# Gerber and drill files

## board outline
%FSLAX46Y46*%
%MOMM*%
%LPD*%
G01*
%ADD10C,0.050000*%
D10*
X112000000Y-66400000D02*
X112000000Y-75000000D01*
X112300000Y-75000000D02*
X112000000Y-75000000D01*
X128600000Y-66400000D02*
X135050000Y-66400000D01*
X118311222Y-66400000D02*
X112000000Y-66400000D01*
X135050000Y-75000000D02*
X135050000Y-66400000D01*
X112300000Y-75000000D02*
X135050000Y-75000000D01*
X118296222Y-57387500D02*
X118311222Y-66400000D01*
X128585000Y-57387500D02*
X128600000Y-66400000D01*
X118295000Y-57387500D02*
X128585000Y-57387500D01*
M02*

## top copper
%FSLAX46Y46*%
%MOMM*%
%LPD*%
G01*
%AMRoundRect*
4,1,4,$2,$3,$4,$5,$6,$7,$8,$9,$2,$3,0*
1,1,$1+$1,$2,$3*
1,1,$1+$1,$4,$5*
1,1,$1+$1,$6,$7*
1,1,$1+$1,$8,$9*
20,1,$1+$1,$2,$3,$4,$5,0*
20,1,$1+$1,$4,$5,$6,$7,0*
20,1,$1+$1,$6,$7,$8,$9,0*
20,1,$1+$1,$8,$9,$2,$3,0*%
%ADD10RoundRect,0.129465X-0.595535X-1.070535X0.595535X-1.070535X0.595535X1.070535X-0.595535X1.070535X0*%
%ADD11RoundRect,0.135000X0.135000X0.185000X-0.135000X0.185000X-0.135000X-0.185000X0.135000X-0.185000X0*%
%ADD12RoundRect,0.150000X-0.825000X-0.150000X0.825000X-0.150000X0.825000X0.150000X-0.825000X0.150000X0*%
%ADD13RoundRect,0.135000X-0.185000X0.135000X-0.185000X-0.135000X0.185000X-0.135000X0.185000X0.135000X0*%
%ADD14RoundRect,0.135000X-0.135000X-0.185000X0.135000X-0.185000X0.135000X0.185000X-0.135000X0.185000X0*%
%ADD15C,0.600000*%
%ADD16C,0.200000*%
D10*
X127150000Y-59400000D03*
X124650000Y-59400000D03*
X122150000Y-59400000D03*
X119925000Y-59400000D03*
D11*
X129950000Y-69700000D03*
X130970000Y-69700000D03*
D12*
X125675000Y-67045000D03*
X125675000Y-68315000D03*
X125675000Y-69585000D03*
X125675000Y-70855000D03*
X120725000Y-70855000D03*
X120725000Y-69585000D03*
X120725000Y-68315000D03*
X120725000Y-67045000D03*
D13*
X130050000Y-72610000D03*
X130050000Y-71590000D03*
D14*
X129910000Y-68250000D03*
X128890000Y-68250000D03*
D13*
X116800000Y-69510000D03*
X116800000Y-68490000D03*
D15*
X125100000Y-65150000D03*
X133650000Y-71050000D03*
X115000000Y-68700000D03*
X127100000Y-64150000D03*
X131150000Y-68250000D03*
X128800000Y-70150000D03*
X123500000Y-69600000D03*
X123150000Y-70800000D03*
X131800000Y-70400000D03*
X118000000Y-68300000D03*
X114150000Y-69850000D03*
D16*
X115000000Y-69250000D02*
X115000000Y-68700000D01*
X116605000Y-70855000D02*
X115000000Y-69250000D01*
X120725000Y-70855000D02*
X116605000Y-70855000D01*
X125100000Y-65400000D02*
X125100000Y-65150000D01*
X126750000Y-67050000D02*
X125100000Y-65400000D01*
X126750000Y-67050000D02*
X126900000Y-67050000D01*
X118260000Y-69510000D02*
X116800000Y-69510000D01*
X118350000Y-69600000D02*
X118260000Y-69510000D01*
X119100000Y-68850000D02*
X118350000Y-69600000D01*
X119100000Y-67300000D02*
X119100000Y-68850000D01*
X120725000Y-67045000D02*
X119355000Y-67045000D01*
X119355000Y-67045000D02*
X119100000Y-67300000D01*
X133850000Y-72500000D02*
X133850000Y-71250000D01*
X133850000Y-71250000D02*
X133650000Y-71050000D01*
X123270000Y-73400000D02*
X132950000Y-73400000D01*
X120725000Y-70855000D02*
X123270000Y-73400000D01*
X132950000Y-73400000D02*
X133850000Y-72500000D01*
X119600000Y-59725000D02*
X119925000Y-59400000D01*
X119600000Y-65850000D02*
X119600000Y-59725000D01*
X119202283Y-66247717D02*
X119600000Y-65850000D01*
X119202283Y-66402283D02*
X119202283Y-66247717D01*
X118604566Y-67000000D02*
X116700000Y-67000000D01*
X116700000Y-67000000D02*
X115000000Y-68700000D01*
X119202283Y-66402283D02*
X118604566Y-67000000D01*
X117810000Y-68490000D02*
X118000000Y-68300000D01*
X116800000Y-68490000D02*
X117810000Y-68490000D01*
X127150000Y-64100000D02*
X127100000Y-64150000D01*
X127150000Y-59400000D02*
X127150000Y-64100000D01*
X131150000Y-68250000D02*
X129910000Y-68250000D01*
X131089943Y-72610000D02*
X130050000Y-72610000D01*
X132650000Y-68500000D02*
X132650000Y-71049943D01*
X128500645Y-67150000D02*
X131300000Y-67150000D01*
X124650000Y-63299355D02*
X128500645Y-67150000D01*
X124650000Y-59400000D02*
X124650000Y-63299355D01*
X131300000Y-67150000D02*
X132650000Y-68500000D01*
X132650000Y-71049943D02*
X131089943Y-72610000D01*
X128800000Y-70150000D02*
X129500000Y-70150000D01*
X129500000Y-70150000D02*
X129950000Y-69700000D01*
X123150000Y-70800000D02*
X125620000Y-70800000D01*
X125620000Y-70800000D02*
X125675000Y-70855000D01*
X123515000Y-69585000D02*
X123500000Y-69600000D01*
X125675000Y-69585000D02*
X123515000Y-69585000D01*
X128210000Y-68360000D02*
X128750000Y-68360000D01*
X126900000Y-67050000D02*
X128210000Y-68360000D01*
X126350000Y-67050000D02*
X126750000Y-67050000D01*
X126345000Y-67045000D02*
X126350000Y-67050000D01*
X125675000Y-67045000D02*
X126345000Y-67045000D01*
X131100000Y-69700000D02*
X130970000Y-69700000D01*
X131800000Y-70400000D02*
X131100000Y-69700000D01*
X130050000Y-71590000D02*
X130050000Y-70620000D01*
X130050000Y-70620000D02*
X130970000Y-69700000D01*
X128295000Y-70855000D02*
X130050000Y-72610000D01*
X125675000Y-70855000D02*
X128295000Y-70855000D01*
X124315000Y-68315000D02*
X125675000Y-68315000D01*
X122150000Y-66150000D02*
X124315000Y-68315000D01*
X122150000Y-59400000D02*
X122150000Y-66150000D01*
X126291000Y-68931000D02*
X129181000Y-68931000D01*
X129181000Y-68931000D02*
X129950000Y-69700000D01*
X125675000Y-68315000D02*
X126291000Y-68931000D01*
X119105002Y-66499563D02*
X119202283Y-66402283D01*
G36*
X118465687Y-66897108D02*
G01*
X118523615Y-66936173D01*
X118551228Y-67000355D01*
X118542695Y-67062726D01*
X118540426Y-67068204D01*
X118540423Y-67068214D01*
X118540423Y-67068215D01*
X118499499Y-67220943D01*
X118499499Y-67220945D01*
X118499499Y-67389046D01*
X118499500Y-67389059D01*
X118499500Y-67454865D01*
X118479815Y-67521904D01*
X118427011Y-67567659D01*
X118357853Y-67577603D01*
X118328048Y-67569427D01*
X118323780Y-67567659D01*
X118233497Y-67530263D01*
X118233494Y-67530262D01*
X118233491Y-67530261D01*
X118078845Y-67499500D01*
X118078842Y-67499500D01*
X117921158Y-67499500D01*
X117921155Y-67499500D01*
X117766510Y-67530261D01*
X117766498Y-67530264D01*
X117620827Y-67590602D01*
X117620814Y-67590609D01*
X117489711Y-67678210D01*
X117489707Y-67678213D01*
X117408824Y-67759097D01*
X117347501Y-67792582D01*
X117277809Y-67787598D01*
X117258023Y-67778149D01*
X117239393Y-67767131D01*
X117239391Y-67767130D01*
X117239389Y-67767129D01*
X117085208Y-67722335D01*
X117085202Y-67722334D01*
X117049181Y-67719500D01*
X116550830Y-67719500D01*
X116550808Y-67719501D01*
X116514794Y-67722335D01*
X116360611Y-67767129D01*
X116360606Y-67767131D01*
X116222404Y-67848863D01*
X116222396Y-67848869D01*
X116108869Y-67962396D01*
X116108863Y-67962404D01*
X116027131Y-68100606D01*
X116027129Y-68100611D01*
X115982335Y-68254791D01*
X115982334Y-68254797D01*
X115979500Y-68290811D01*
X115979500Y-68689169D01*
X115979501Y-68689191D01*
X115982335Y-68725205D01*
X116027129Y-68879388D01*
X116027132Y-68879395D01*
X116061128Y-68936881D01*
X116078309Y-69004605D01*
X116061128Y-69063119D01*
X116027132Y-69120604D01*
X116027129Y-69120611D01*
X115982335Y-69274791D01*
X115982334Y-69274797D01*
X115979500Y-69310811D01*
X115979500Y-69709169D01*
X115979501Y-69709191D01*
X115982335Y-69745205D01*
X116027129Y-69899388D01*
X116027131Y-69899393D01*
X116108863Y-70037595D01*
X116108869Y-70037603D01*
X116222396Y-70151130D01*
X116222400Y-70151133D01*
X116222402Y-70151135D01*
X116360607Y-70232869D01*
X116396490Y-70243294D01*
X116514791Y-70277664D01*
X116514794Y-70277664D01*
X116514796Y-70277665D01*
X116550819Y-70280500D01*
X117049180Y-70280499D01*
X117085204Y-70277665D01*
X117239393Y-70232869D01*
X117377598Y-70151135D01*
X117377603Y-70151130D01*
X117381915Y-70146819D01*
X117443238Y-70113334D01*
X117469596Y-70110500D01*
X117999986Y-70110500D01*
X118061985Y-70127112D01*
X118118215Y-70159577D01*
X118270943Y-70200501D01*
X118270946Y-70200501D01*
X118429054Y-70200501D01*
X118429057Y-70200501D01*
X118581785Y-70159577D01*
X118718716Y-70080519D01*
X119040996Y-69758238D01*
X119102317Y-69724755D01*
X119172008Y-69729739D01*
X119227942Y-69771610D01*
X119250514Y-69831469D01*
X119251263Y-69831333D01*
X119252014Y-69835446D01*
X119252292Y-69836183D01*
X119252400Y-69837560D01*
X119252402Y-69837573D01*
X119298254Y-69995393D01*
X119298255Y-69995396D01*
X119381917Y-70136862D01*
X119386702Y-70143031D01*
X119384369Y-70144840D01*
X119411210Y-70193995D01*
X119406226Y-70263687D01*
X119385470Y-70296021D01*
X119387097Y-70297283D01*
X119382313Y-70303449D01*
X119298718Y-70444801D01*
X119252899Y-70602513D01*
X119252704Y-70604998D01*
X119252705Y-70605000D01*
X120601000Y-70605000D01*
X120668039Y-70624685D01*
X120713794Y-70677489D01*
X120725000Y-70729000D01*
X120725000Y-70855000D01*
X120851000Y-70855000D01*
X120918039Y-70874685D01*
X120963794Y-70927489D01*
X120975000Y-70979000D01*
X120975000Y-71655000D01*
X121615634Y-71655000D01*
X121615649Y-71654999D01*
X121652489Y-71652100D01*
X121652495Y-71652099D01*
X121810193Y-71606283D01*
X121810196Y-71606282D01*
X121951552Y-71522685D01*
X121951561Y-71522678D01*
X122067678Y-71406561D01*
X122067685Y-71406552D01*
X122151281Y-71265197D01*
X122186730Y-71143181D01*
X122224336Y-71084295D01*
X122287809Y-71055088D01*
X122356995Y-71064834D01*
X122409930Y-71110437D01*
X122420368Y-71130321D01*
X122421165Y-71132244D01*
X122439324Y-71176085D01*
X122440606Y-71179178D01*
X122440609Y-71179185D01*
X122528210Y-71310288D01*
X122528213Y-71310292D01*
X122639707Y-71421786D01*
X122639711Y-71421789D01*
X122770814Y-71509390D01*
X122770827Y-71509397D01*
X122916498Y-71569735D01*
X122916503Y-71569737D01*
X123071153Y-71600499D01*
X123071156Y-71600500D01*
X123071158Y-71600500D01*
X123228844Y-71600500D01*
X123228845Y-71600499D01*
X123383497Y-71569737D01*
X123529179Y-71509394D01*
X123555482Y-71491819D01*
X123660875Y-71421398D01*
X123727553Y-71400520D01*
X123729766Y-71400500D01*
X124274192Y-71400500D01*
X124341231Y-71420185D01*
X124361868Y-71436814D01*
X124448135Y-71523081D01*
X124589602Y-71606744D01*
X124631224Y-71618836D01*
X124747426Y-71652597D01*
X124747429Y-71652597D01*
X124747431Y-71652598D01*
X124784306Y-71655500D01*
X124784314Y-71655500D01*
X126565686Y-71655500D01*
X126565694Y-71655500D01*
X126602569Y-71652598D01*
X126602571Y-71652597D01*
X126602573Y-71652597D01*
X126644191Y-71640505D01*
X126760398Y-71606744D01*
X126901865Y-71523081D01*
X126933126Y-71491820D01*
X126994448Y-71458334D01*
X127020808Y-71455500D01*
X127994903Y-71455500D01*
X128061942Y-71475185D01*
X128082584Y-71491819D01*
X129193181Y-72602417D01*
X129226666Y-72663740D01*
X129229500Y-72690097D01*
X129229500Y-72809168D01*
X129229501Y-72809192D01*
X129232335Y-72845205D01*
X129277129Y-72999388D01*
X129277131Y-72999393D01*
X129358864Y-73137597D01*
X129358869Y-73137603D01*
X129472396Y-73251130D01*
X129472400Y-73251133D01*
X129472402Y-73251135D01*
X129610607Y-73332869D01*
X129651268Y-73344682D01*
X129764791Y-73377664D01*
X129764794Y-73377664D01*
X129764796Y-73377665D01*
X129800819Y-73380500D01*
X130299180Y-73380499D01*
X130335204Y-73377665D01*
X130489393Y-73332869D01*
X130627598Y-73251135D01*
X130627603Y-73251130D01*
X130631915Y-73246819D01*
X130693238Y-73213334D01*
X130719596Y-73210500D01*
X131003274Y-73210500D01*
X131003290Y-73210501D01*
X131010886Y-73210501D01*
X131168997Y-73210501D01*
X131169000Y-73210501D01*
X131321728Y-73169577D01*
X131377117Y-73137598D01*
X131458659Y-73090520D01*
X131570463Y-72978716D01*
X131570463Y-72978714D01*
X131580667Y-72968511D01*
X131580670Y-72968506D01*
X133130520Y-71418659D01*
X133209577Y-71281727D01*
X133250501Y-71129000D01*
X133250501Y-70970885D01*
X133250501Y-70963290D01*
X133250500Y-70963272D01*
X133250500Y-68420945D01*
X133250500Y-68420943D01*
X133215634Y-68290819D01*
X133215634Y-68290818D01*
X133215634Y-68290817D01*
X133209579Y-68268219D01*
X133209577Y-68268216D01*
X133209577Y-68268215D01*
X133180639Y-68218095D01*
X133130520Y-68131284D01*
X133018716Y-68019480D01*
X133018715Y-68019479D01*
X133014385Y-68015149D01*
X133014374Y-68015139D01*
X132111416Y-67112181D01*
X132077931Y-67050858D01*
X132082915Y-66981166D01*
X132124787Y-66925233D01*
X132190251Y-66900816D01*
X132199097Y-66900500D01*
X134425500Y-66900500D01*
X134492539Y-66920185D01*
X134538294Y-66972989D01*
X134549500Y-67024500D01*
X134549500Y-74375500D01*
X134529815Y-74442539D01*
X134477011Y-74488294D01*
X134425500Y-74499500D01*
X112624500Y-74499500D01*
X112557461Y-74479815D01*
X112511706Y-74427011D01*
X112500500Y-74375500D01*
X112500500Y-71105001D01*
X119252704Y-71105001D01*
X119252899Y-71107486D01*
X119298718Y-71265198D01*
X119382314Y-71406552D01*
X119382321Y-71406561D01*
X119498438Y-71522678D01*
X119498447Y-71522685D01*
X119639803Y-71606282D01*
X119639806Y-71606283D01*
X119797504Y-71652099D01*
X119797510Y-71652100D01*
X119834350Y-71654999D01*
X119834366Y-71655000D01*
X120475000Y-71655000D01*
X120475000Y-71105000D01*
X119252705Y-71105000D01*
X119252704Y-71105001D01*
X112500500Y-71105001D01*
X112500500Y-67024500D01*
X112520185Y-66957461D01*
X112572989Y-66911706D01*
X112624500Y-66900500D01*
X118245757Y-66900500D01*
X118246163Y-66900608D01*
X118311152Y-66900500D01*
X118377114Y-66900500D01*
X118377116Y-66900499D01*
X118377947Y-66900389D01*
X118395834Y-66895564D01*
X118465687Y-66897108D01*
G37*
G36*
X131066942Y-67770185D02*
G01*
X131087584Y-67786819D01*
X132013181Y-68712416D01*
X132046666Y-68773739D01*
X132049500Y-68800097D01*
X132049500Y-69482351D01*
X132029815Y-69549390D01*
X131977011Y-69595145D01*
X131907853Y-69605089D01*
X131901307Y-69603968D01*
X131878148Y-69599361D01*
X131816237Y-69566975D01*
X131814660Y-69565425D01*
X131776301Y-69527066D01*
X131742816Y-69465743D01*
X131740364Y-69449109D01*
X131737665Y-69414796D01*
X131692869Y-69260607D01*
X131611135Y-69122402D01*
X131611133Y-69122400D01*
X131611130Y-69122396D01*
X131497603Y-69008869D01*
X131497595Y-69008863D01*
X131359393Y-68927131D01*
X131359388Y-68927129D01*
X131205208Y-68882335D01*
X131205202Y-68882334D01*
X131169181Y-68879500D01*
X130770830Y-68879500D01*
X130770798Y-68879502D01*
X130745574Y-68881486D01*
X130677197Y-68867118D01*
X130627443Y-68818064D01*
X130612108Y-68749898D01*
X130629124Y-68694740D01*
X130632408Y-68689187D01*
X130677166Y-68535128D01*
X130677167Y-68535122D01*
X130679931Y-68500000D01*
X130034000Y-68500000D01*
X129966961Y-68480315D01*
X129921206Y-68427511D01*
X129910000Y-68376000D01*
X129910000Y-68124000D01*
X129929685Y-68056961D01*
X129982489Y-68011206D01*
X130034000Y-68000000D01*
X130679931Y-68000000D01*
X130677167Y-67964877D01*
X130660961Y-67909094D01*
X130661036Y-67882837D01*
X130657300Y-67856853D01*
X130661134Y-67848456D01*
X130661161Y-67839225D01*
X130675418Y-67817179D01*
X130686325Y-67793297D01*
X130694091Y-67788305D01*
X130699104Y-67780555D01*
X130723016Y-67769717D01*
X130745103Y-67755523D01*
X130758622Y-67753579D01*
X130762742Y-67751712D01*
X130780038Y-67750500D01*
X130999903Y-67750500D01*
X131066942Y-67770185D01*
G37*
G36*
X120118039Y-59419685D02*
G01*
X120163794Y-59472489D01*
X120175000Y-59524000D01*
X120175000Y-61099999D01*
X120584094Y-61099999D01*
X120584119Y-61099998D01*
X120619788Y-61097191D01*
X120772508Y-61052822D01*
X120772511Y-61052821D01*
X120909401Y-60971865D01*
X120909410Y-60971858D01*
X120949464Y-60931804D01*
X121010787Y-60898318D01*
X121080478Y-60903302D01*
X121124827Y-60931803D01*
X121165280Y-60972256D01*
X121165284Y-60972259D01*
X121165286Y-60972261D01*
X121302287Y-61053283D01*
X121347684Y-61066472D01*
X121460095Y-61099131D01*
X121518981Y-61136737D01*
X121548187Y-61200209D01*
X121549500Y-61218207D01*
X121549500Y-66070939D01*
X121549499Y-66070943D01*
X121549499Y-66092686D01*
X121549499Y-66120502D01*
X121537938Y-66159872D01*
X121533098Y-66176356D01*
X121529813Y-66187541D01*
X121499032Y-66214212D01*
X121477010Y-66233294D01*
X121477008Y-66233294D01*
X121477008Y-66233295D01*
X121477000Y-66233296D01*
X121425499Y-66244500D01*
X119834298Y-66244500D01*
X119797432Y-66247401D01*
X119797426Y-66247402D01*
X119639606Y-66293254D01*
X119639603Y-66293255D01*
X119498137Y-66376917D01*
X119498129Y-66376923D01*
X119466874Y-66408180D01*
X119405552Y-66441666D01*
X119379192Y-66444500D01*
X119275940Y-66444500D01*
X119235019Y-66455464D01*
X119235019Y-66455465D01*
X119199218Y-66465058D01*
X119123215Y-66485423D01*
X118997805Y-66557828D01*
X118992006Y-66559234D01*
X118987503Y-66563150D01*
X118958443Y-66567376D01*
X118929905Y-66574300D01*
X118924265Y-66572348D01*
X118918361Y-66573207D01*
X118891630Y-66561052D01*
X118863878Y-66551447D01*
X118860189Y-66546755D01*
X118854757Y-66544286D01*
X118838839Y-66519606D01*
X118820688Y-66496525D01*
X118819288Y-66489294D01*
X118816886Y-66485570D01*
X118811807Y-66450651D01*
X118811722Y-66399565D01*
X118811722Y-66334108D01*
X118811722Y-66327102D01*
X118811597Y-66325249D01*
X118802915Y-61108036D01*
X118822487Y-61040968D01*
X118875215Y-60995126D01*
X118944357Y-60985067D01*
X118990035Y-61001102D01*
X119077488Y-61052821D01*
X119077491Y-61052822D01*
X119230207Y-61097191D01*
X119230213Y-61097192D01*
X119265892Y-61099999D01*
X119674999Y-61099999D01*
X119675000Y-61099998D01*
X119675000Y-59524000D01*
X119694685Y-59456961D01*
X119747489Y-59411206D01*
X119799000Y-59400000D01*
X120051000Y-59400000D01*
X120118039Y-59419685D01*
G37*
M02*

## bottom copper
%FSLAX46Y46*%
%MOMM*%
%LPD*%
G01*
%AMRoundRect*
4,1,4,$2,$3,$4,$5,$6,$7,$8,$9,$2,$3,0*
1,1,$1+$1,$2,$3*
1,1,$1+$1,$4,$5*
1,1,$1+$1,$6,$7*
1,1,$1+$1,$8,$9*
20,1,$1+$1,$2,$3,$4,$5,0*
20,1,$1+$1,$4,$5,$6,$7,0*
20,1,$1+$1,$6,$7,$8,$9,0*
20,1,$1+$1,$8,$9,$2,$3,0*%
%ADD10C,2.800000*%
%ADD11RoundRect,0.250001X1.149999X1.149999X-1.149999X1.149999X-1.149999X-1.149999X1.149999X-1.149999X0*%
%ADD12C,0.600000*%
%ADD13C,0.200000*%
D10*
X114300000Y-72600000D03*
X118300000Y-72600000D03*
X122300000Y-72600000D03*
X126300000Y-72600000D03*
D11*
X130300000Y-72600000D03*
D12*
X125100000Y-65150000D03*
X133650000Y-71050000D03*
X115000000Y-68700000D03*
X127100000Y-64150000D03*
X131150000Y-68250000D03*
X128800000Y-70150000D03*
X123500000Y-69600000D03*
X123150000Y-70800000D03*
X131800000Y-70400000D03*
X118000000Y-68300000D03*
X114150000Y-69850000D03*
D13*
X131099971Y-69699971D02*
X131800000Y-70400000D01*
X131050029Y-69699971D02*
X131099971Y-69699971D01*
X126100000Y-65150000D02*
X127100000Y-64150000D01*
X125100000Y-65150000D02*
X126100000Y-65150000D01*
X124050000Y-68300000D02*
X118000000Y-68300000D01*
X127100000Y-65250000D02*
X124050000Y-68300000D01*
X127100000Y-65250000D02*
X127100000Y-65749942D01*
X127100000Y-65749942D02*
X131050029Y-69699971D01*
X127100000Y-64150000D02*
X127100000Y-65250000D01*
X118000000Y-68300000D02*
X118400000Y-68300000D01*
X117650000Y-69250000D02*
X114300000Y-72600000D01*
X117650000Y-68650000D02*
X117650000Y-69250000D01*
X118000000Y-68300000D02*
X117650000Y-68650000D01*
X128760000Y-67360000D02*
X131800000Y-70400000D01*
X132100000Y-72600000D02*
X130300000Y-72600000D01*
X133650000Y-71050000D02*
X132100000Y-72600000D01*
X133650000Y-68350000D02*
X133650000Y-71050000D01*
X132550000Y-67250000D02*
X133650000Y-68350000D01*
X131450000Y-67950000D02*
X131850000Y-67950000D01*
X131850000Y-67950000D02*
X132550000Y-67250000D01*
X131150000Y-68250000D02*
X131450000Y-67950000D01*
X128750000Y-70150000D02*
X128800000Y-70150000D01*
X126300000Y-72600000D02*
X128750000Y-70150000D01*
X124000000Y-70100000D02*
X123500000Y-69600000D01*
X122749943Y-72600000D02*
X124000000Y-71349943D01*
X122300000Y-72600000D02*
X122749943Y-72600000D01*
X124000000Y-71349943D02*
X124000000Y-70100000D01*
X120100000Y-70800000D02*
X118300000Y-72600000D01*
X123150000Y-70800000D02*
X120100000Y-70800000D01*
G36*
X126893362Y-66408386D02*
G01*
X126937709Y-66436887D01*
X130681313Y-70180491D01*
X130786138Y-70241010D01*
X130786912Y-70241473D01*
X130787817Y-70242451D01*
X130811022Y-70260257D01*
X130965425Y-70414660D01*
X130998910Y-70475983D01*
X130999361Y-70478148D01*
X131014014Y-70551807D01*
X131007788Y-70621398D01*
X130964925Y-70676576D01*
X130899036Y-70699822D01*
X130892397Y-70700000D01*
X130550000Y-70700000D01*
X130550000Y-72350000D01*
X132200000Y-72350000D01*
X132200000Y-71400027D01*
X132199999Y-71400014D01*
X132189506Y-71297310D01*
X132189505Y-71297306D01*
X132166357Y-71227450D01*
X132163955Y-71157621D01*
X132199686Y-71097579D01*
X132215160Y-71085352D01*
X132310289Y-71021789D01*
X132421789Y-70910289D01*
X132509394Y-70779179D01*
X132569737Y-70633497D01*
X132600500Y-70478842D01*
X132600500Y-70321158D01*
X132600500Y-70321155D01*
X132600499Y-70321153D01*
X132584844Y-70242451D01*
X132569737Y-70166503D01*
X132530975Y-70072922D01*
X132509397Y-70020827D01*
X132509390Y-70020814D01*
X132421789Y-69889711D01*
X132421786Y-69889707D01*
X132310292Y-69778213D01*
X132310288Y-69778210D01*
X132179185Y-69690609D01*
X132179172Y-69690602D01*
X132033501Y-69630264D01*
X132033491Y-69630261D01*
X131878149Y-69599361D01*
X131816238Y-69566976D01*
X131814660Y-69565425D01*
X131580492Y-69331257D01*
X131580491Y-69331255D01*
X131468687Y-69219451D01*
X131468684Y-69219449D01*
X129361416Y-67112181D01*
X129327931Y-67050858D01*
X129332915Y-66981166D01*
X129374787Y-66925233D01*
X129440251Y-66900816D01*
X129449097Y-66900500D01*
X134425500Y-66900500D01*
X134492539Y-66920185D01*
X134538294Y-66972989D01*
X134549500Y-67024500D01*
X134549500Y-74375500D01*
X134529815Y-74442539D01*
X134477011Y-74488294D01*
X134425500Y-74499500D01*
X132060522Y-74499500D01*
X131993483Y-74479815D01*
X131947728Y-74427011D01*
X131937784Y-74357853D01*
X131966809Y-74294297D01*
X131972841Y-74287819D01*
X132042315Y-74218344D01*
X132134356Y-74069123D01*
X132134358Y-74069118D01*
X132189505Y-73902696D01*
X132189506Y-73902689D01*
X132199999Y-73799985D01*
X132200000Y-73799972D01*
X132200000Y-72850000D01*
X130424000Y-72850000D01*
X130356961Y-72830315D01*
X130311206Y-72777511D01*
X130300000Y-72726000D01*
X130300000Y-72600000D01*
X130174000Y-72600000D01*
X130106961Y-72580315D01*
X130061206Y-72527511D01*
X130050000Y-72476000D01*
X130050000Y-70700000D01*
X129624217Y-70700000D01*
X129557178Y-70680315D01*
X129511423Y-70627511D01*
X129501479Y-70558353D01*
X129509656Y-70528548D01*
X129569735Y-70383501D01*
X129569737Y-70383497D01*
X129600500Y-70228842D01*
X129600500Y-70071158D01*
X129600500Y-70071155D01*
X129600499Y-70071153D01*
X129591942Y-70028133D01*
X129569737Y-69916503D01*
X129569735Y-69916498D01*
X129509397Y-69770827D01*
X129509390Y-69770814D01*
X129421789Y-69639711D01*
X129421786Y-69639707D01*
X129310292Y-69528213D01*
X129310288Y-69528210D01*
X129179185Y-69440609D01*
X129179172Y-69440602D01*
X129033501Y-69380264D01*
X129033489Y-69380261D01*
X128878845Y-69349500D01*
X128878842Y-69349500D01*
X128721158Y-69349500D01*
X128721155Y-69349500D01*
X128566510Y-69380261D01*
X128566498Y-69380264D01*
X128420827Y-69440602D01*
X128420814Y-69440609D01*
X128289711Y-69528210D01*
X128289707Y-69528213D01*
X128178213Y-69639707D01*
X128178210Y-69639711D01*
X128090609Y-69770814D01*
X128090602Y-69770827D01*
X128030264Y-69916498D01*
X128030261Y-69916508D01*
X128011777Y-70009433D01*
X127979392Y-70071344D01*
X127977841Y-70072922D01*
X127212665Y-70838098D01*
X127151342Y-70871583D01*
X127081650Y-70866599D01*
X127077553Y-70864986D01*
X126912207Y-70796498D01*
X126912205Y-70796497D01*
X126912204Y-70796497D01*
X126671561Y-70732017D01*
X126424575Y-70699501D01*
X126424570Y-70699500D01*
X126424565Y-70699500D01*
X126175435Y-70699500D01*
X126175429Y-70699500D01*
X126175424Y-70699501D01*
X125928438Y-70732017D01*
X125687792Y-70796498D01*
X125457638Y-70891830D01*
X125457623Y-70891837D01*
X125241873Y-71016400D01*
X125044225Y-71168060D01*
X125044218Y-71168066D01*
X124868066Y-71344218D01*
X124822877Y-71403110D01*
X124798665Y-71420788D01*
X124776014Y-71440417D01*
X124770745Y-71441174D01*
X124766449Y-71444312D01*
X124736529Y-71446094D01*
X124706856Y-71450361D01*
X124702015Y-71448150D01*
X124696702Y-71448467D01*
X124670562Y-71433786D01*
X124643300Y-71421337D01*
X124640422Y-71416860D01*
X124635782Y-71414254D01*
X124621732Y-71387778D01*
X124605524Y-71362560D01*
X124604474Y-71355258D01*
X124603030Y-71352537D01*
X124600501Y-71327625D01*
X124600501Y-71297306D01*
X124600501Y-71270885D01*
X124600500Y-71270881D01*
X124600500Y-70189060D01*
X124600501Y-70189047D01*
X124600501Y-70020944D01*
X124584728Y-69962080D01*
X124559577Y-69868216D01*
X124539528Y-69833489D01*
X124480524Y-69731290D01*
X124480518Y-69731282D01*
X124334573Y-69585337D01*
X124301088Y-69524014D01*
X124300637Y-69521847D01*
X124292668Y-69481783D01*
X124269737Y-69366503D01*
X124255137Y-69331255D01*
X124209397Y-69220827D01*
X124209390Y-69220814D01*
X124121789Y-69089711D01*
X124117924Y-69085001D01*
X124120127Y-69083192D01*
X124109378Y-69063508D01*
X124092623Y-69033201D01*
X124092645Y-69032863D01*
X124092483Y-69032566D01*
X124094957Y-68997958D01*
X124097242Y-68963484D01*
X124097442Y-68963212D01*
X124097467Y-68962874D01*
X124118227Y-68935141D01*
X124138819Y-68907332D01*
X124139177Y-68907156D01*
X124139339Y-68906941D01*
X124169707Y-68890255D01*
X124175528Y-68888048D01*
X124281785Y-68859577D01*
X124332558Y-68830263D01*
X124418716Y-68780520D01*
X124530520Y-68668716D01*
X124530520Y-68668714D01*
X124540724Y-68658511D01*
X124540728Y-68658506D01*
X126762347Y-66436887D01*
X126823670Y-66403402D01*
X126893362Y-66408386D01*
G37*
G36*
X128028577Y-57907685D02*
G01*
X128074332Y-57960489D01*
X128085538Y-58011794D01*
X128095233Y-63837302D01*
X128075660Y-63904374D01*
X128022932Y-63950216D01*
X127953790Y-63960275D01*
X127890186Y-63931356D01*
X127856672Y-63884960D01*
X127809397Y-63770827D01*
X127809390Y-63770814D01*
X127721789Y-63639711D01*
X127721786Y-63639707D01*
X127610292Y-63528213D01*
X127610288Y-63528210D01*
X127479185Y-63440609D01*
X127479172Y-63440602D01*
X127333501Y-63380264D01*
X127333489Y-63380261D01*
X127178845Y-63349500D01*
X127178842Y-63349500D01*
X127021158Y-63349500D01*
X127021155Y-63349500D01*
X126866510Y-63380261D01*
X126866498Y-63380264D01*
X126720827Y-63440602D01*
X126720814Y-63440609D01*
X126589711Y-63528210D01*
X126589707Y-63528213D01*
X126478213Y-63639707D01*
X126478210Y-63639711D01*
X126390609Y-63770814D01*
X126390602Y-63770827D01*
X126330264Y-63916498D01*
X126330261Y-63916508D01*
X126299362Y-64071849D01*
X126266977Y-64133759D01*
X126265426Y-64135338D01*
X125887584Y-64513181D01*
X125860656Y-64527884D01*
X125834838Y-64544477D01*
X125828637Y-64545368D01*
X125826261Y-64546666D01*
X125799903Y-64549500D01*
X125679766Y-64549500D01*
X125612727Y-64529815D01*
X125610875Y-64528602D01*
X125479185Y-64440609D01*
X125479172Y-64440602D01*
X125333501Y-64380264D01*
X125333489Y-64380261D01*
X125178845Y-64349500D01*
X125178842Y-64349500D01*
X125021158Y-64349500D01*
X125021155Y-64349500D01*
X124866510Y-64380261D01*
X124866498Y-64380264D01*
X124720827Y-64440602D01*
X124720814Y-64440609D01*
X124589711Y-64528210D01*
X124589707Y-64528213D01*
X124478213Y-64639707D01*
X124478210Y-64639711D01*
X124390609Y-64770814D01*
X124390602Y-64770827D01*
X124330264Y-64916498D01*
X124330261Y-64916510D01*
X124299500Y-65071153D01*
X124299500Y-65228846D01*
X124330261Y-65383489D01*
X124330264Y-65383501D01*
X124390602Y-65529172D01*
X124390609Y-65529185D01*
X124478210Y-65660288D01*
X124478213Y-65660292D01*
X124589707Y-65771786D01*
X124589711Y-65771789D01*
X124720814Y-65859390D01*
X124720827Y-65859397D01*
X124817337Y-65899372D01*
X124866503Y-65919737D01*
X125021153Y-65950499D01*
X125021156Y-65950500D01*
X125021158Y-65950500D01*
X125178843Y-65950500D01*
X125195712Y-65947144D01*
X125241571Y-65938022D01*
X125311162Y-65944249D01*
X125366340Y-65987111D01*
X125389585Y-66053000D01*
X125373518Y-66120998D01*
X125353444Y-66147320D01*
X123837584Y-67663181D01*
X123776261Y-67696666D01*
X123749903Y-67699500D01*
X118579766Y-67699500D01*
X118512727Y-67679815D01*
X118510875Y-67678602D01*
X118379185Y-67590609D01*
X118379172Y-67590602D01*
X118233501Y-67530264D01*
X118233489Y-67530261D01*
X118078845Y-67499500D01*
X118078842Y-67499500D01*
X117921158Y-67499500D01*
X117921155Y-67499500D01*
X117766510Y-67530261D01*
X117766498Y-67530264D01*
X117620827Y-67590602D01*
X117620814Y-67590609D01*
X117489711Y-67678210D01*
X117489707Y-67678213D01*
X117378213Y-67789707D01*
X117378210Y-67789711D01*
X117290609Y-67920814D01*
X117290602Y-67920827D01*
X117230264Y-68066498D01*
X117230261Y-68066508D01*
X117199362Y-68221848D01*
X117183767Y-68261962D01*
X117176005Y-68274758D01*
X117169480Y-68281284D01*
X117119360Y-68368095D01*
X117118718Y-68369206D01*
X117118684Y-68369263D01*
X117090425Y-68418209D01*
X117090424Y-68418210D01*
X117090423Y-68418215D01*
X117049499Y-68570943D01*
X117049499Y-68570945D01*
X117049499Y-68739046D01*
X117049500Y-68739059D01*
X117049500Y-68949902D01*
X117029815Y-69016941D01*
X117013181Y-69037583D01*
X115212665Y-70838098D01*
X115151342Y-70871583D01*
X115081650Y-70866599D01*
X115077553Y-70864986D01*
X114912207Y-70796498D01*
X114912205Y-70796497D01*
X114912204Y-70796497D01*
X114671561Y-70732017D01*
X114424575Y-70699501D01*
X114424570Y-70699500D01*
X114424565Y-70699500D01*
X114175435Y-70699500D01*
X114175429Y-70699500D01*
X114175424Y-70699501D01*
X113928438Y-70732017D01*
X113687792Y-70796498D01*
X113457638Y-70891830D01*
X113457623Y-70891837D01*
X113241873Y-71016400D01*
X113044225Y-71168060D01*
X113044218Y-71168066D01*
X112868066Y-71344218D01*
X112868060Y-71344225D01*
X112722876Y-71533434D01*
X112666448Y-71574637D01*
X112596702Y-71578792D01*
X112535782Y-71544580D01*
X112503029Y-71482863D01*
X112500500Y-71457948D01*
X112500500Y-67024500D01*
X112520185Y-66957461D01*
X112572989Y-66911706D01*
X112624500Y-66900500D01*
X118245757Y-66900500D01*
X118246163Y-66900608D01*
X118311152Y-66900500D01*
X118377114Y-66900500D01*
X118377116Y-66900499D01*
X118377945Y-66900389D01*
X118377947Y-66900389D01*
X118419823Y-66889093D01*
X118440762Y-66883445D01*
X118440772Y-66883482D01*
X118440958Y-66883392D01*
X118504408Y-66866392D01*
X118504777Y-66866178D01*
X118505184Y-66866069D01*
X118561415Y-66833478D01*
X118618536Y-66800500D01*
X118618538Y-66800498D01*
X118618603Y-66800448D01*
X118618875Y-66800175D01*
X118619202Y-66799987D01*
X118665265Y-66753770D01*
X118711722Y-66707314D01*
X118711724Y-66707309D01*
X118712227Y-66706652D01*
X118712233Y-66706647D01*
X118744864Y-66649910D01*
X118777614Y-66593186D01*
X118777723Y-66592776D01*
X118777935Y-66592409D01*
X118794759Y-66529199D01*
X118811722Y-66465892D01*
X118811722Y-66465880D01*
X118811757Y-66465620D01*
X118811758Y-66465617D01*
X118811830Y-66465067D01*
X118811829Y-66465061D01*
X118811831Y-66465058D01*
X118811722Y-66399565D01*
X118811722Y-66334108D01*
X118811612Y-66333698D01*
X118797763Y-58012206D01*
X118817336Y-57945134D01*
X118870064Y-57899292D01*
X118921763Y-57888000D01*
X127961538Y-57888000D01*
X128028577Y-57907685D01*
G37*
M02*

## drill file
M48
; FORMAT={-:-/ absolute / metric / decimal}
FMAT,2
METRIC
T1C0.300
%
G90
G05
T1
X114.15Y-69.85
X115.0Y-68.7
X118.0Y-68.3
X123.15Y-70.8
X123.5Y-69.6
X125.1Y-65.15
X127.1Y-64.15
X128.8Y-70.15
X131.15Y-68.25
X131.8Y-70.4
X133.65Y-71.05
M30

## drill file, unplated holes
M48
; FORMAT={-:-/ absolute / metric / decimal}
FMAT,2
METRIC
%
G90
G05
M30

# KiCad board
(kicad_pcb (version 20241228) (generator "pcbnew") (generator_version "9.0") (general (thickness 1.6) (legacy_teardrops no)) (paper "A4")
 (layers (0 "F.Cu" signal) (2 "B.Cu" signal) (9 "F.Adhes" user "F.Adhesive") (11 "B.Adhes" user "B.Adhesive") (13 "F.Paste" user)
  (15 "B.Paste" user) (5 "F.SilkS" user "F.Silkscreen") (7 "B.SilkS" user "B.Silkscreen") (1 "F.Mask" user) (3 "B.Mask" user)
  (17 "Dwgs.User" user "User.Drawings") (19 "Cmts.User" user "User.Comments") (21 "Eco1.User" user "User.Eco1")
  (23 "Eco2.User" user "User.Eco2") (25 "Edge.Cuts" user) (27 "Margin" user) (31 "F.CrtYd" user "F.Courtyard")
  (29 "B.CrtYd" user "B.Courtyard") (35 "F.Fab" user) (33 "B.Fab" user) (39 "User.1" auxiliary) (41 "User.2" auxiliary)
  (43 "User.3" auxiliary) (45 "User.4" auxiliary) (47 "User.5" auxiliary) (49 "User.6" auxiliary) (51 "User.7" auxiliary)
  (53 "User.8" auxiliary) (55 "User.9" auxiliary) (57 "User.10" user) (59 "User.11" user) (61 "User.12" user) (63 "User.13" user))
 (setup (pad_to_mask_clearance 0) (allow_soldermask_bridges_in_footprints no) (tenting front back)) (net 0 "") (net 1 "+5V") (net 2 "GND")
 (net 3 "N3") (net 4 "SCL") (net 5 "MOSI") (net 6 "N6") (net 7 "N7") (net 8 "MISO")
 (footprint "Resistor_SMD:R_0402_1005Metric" (layer "F.Cu") (at 129.4 68.25)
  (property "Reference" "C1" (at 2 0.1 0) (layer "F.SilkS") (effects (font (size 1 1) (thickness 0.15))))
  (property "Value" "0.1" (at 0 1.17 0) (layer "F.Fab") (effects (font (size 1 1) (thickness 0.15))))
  (pad "1" smd roundrect (at -0.51 0) (size 0.54 0.64) (layers "F.Cu" "F.Mask" "F.Paste") (roundrect_rratio 0.25) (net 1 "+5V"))
  (pad "2" smd roundrect (at 0.51 0) (size 0.54 0.64) (layers "F.Cu" "F.Mask" "F.Paste") (roundrect_rratio 0.25) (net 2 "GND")))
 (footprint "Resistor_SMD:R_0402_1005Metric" (layer "F.Cu") (at 116.8 69 -90)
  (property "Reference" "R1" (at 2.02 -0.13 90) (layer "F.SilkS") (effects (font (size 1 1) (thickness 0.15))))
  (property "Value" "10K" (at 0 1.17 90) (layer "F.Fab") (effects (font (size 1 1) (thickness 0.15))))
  (pad "1" smd roundrect (at -0.51 0 270) (size 0.54 0.64) (layers "F.Cu" "F.Mask" "F.Paste") (roundrect_rratio 0.25) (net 1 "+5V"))
  (pad "2" smd roundrect (at 0.51 0 270) (size 0.54 0.64) (layers "F.Cu" "F.Mask" "F.Paste") (roundrect_rratio 0.25) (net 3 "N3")))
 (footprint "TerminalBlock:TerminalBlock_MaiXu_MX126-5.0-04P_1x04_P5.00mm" (layer "F.Cu") (at 120.15 59.4)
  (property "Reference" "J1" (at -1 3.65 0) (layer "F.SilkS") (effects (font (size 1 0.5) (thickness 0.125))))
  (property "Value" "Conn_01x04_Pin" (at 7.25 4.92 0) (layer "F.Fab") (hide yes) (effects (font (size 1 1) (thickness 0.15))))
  (pad "1" smd roundrect (at -0.225 0) (size 1.45 2.4) (layers "F.Cu" "F.Mask" "F.Paste") (roundrect_rratio 0.089286) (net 2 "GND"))
  (pad "2" smd roundrect (at 2 0) (size 1.45 2.4) (layers "F.Cu" "F.Mask" "F.Paste") (roundrect_rratio 0.089286) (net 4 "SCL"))
  (pad "3" smd roundrect (at 4.5 0) (size 1.45 2.4) (layers "F.Cu" "F.Mask" "F.Paste") (roundrect_rratio 0.089286) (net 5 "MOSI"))
  (pad "4" smd roundrect (at 7 0) (size 1.45 2.4) (layers "F.Cu" "F.Mask" "F.Paste") (roundrect_rratio 0.089286) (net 1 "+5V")))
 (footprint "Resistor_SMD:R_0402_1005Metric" (layer "F.Cu") (at 130.46 69.7 180)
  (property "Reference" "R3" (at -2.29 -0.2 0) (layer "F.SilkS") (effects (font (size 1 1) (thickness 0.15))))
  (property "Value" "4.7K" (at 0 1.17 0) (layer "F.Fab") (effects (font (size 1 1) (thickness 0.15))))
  (pad "1" smd roundrect (at -0.51 0 180) (size 0.54 0.64) (layers "F.Cu" "F.Mask" "F.Paste") (roundrect_rratio 0.25) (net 1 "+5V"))
  (pad "2" smd roundrect (at 0.51 0 180) (size 0.54 0.64) (layers "F.Cu" "F.Mask" "F.Paste") (roundrect_rratio 0.25) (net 4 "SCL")))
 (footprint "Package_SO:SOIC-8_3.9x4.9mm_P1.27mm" (layer "F.Cu") (at 123.2 68.95)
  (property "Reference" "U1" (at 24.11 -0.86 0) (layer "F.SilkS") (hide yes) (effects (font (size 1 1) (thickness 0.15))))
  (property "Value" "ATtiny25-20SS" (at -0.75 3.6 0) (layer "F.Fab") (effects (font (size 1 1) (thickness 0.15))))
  (pad "1" smd roundrect (at -2.475 -1.905) (size 1.95 0.6) (layers "F.Cu" "F.Mask" "F.Paste") (roundrect_rratio 0.25) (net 3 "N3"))
  (pad "2" smd roundrect (at -2.475 -0.635) (size 1.95 0.6) (layers "F.Cu" "F.Mask" "F.Paste") (roundrect_rratio 0.25) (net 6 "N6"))
  (pad "3" smd roundrect (at -2.475 0.635) (size 1.95 0.6) (layers "F.Cu" "F.Mask" "F.Paste") (roundrect_rratio 0.25) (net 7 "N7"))
  (pad "4" smd roundrect (at -2.475 1.905) (size 1.95 0.6) (layers "F.Cu" "F.Mask" "F.Paste") (roundrect_rratio 0.25) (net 2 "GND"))
  (pad "5" smd roundrect (at 2.475 1.905) (size 1.95 0.6) (layers "F.Cu" "F.Mask" "F.Paste") (roundrect_rratio 0.25) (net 5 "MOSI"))
  (pad "6" smd roundrect (at 2.475 0.635) (size 1.95 0.6) (layers "F.Cu" "F.Mask" "F.Paste") (roundrect_rratio 0.25) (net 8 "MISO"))
  (pad "7" smd roundrect (at 2.475 -0.635) (size 1.95 0.6) (layers "F.Cu" "F.Mask" "F.Paste") (roundrect_rratio 0.25) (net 4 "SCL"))
  (pad "8" smd roundrect (at 2.475 -1.905) (size 1.95 0.6) (layers "F.Cu" "F.Mask" "F.Paste") (roundrect_rratio 0.25) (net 1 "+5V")))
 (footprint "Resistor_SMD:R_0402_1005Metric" (layer "F.Cu") (at 130.05 72.1 -90)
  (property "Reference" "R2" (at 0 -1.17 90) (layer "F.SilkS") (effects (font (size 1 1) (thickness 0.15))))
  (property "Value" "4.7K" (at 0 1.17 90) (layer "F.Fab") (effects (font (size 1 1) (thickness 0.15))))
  (pad "1" smd roundrect (at -0.51 0 270) (size 0.54 0.64) (layers "F.Cu" "F.Mask" "F.Paste") (roundrect_rratio 0.25) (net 1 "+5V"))
  (pad "2" smd roundrect (at 0.51 0 270) (size 0.54 0.64) (layers "F.Cu" "F.Mask" "F.Paste") (roundrect_rratio 0.25) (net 5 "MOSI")))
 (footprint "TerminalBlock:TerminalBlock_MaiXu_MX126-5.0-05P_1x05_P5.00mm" (layer "B.Cu") (at 131.3 72.6 180)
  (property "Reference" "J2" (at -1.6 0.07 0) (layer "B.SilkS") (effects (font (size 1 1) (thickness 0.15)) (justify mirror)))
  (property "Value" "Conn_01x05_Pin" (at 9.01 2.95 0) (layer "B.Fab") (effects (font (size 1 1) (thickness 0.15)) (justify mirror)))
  (pad "1" smd roundrect (at 1 0 180) (size 2.8 2.8) (layers "B.Cu" "B.Mask" "B.Paste") (roundrect_rratio 0.089286) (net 2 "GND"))
  (pad "2" smd circle (at 5 0 180) (size 2.8 2.8) (layers "B.Cu" "B.Mask" "B.Paste") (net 4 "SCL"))
  (pad "3" smd circle (at 9 0 180) (size 2.8 2.8) (layers "B.Cu" "B.Mask" "B.Paste") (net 8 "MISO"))
  (pad "4" smd circle (at 13 0 180) (size 2.8 2.8) (layers "B.Cu" "B.Mask" "B.Paste") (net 5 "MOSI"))
  (pad "5" smd circle (at 17 0 180) (size 2.8 2.8) (layers "B.Cu" "B.Mask" "B.Paste") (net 1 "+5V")))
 (gr_line (start 118.295 57.3875) (end 128.585 57.3875) (stroke (width 0.05) (type default)) (layer "Edge.Cuts"))
 (gr_line (start 118.311222 66.4) (end 112 66.4) (stroke (width 0.05) (type default)) (layer "Edge.Cuts"))
 (gr_line (start 112 66.4) (end 112 75) (stroke (width 0.05) (type default)) (layer "Edge.Cuts"))
 (gr_line (start 128.585 57.3875) (end 128.6 66.4) (stroke (width 0.05) (type default)) (layer "Edge.Cuts"))
 (gr_line (start 128.6 66.4) (end 135.05 66.4) (stroke (width 0.05) (type default)) (layer "Edge.Cuts"))
 (gr_line (start 112.3 75) (end 112 75) (stroke (width 0.05) (type default)) (layer "Edge.Cuts"))
 (gr_line (start 118.296222 57.3875) (end 118.311222 66.4) (stroke (width 0.05) (type default)) (layer "Edge.Cuts"))
 (gr_line (start 135.05 75) (end 135.05 66.4) (stroke (width 0.05) (type default)) (layer "Edge.Cuts"))
 (gr_line (start 112.3 75) (end 135.05 75) (stroke (width 0.05) (type default)) (layer "Edge.Cuts"))
 (segment (start 119.202283 66.402283) (end 119.202283 66.247717) (width 0.2) (layer "F.Cu") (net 2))
 (segment (start 119.6 59.725) (end 119.925 59.4) (width 0.2) (layer "F.Cu") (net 2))
 (segment (start 123.27 73.4) (end 132.95 73.4) (width 0.2) (layer "F.Cu") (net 2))
 (segment (start 115 69.25) (end 115 68.7) (width 0.2) (layer "F.Cu") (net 2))
 (segment (start 120.725 70.855) (end 116.605 70.855) (width 0.2) (layer "F.Cu") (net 2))
 (segment (start 119.202283 66.247717) (end 119.6 65.85) (width 0.2) (layer "F.Cu") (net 2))
 (segment (start 119.6 65.85) (end 119.6 59.725) (width 0.2) (layer "F.Cu") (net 2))
 (segment (start 133.85 72.5) (end 133.85 71.25) (width 0.2) (layer "F.Cu") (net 2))
 (segment (start 131.15 68.25) (end 129.91 68.25) (width 0.2) (layer "F.Cu") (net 2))
 (segment (start 118.604566 67) (end 116.7 67) (width 0.2) (layer "F.Cu") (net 2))
 (segment (start 133.85 71.25) (end 133.65 71.05) (width 0.2) (layer "F.Cu") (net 2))
 (segment (start 116.7 67) (end 115 68.7) (width 0.2) (layer "F.Cu") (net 2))
 (segment (start 120.725 70.855) (end 123.27 73.4) (width 0.2) (layer "F.Cu") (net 2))
 (segment (start 116.605 70.855) (end 115 69.25) (width 0.2) (layer "F.Cu") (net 2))
 (segment (start 119.202283 66.402283) (end 118.604566 67) (width 0.2) (layer "F.Cu") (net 2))
 (segment (start 132.95 73.4) (end 133.85 72.5) (width 0.2) (layer "F.Cu") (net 2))
 (segment (start 119.105002 66.499563) (end 119.202283 66.402283) (width 0.2) (layer "F.Cu") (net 2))
 (via (at 131.15 68.25) (size 0.6) (drill 0.3) (layers "F.Cu" "B.Cu") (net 2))
 (via (at 114.15 69.85) (size 0.6) (drill 0.3) (layers "F.Cu" "B.Cu") (free yes) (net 2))
 (via (at 115 68.7) (size 0.6) (drill 0.3) (layers "F.Cu" "B.Cu") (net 2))
 (via (at 133.65 71.05) (size 0.6) (drill 0.3) (layers "F.Cu" "B.Cu") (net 2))
 (segment (start 133.65 68.35) (end 133.65 71.05) (width 0.2) (layer "B.Cu") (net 2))
 (segment (start 132.55 67.25) (end 133.65 68.35) (width 0.2) (layer "B.Cu") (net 2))
 (segment (start 132.1 72.6) (end 130.3 72.6) (width 0.2) (layer "B.Cu") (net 2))
 (segment (start 131.45 67.95) (end 131.85 67.95) (width 0.2) (layer "B.Cu") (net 2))
 (segment (start 133.65 71.05) (end 132.1 72.6) (width 0.2) (layer "B.Cu") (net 2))
 (segment (start 131.15 68.25) (end 131.45 67.95) (width 0.2) (layer "B.Cu") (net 2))
 (segment (start 131.85 67.95) (end 132.55 67.25) (width 0.2) (layer "B.Cu") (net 2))
 (segment (start 131.8 70.4) (end 131.1 69.7) (width 0.2) (layer "F.Cu") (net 1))
 (segment (start 125.675 67.045) (end 126.345 67.045) (width 0.2) (layer "F.Cu") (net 1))
 (segment (start 130.05 70.62) (end 130.97 69.7) (width 0.2) (layer "F.Cu") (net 1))
 (segment (start 116.8 68.49) (end 117.81 68.49) (width 0.2) (layer "F.Cu") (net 1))
 (segment (start 127.15 64.1) (end 127.1 64.15) (width 0.2) (layer "F.Cu") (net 1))
 (segment (start 126.75 67.05) (end 126.9 67.05) (width 0.2) (layer "F.Cu") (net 1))
 (segment (start 131.1 69.7) (end 130.97 69.7) (width 0.2) (layer "F.Cu") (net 1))
 (segment (start 125.1 65.4) (end 125.1 65.15) (width 0.2) (layer "F.Cu") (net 1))
 (segment (start 128.21 68.36) (end 128.75 68.36) (width 0.2) (layer "F.Cu") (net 1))
 (segment (start 126.9 67.05) (end 128.21 68.36) (width 0.2) (layer "F.Cu") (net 1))
 (segment (start 130.05 71.59) (end 130.05 70.62) (width 0.2) (layer "F.Cu") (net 1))
 (segment (start 126.75 67.05) (end 125.1 65.4) (width 0.2) (layer "F.Cu") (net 1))
 (segment (start 127.15 59.4) (end 127.15 64.1) (width 0.2) (layer "F.Cu") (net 1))
 (segment (start 126.345 67.045) (end 126.35 67.05) (width 0.2) (layer "F.Cu") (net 1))
 (segment (start 126.35 67.05) (end 126.75 67.05) (width 0.2) (layer "F.Cu") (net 1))
 (segment (start 117.81 68.49) (end 118 68.3) (width 0.2) (layer "F.Cu") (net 1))
 (via (at 127.1 64.15) (size 0.6) (drill 0.3) (layers "F.Cu" "B.Cu") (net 1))
 (via (at 131.8 70.4) (size 0.6) (drill 0.3) (layers "F.Cu" "B.Cu") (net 1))
 (via (at 118 68.3) (size 0.6) (drill 0.3) (layers "F.Cu" "B.Cu") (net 1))
 (via (at 125.1 65.15) (size 0.6) (drill 0.3) (layers "F.Cu" "B.Cu") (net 1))
 (segment (start 118 68.3) (end 117.65 68.65) (width 0.2) (layer "B.Cu") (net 1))
 (segment (start 131.050029 69.699971) (end 131.099971 69.699971) (width 0.2) (layer "B.Cu") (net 1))
 (segment (start 127.1 64.15) (end 127.1 65.25) (width 0.2) (layer "B.Cu") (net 1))
 (segment (start 125.1 65.15) (end 126.1 65.15) (width 0.2) (layer "B.Cu") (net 1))
 (segment (start 118 68.3) (end 118.4 68.3) (width 0.2) (layer "B.Cu") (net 1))
 (segment (start 117.65 68.65) (end 117.65 69.25) (width 0.2) (layer "B.Cu") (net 1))
 (segment (start 124.05 68.3) (end 118 68.3) (width 0.2) (layer "B.Cu") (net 1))
 (segment (start 127.1 65.25) (end 124.05 68.3) (width 0.2) (layer "B.Cu") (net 1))
 (segment (start 117.65 69.25) (end 114.3 72.6) (width 0.2) (layer "B.Cu") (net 1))
 (segment (start 131.099971 69.699971) (end 131.8 70.4) (width 0.2) (layer "B.Cu") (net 1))
 (segment (start 127.1 65.25) (end 127.1 65.749942) (width 0.2) (layer "B.Cu") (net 1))
 (segment (start 127.1 65.749942) (end 131.050029 69.699971) (width 0.2) (layer "B.Cu") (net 1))
 (segment (start 126.1 65.15) (end 127.1 64.15) (width 0.2) (layer "B.Cu") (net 1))
 (segment (start 128.76 67.36) (end 131.8 70.4) (width 0.2) (layer "B.Cu") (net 1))
 (segment (start 128.295 70.855) (end 130.05 72.61) (width 0.2) (layer "F.Cu") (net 5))
 (segment (start 132.65 71.049943) (end 131.089943 72.61) (width 0.2) (layer "F.Cu") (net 5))
 (segment (start 124.65 59.4) (end 124.65 63.299355) (width 0.2) (layer "F.Cu") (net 5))
 (segment (start 131.089943 72.61) (end 130.05 72.61) (width 0.2) (layer "F.Cu") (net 5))
 (segment (start 123.15 70.8) (end 125.62 70.8) (width 0.2) (layer "F.Cu") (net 5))
 (segment (start 132.65 68.5) (end 132.65 71.049943) (width 0.2) (layer "F.Cu") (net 5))
 (segment (start 125.62 70.8) (end 125.675 70.855) (width 0.2) (layer "F.Cu") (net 5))
 (segment (start 131.3 67.15) (end 132.65 68.5) (width 0.2) (layer "F.Cu") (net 5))
 (segment (start 128.500645 67.15) (end 131.3 67.15) (width 0.2) (layer "F.Cu") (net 5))
 (segment (start 124.65 63.299355) (end 128.500645 67.15) (width 0.2) (layer "F.Cu") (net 5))
 (segment (start 125.675 70.855) (end 128.295 70.855) (width 0.2) (layer "F.Cu") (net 5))
 (via (at 123.15 70.8) (size 0.6) (drill 0.3) (layers "F.Cu" "B.Cu") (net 5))
 (segment (start 120.1 70.8) (end 118.3 72.6) (width 0.2) (layer "B.Cu") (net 5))
 (segment (start 123.15 70.8) (end 120.1 70.8) (width 0.2) (layer "B.Cu") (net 5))
 (segment (start 129.5 70.15) (end 129.95 69.7) (width 0.2) (layer "F.Cu") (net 4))
 (segment (start 129.181 68.931) (end 129.95 69.7) (width 0.2) (layer "F.Cu") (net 4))
 (segment (start 122.15 66.15) (end 124.315 68.315) (width 0.2) (layer "F.Cu") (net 4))
 (segment (start 128.8 70.15) (end 129.5 70.15) (width 0.2) (layer "F.Cu") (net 4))
 (segment (start 124.315 68.315) (end 125.675 68.315) (width 0.2) (layer "F.Cu") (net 4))
 (segment (start 126.291 68.931) (end 129.181 68.931) (width 0.2) (layer "F.Cu") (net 4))
 (segment (start 125.675 68.315) (end 126.291 68.931) (width 0.2) (layer "F.Cu") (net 4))
 (segment (start 122.15 59.4) (end 122.15 66.15) (width 0.2) (layer "F.Cu") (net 4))
 (via (at 128.8 70.15) (size 0.6) (drill 0.3) (layers "F.Cu" "B.Cu") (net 4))
 (segment (start 128.75 70.15) (end 128.8 70.15) (width 0.2) (layer "B.Cu") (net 4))
 (segment (start 126.3 72.6) (end 128.75 70.15) (width 0.2) (layer "B.Cu") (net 4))
 (segment (start 125.675 69.585) (end 123.515 69.585) (width 0.2) (layer "F.Cu") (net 8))
 (segment (start 123.515 69.585) (end 123.5 69.6) (width 0.2) (layer "F.Cu") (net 8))
 (via (at 123.5 69.6) (size 0.6) (drill 0.3) (layers "F.Cu" "B.Cu") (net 8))
 (segment (start 122.749943 72.6) (end 124 71.349943) (width 0.2) (layer "B.Cu") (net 8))
 (segment (start 124 71.349943) (end 124 70.1) (width 0.2) (layer "B.Cu") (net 8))
 (segment (start 122.3 72.6) (end 122.749943 72.6) (width 0.2) (layer "B.Cu") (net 8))
 (segment (start 124 70.1) (end 123.5 69.6) (width 0.2) (layer "B.Cu") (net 8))
 (segment (start 119.355 67.045) (end 119.1 67.3) (width 0.2) (layer "F.Cu") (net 3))
 (segment (start 119.1 68.85) (end 118.35 69.6) (width 0.2) (layer "F.Cu") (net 3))
 (segment (start 118.35 69.6) (end 118.26 69.51) (width 0.2) (layer "F.Cu") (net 3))
 (segment (start 120.725 67.045) (end 119.355 67.045) (width 0.2) (layer "F.Cu") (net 3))
 (segment (start 118.26 69.51) (end 116.8 69.51) (width 0.2) (layer "F.Cu") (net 3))
 (segment (start 119.1 67.3) (end 119.1 68.85) (width 0.2) (layer "F.Cu") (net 3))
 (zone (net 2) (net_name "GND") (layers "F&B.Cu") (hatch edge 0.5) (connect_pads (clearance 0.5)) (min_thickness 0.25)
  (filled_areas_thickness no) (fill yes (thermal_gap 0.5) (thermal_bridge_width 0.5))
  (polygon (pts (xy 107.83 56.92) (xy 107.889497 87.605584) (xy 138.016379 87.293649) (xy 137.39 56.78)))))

